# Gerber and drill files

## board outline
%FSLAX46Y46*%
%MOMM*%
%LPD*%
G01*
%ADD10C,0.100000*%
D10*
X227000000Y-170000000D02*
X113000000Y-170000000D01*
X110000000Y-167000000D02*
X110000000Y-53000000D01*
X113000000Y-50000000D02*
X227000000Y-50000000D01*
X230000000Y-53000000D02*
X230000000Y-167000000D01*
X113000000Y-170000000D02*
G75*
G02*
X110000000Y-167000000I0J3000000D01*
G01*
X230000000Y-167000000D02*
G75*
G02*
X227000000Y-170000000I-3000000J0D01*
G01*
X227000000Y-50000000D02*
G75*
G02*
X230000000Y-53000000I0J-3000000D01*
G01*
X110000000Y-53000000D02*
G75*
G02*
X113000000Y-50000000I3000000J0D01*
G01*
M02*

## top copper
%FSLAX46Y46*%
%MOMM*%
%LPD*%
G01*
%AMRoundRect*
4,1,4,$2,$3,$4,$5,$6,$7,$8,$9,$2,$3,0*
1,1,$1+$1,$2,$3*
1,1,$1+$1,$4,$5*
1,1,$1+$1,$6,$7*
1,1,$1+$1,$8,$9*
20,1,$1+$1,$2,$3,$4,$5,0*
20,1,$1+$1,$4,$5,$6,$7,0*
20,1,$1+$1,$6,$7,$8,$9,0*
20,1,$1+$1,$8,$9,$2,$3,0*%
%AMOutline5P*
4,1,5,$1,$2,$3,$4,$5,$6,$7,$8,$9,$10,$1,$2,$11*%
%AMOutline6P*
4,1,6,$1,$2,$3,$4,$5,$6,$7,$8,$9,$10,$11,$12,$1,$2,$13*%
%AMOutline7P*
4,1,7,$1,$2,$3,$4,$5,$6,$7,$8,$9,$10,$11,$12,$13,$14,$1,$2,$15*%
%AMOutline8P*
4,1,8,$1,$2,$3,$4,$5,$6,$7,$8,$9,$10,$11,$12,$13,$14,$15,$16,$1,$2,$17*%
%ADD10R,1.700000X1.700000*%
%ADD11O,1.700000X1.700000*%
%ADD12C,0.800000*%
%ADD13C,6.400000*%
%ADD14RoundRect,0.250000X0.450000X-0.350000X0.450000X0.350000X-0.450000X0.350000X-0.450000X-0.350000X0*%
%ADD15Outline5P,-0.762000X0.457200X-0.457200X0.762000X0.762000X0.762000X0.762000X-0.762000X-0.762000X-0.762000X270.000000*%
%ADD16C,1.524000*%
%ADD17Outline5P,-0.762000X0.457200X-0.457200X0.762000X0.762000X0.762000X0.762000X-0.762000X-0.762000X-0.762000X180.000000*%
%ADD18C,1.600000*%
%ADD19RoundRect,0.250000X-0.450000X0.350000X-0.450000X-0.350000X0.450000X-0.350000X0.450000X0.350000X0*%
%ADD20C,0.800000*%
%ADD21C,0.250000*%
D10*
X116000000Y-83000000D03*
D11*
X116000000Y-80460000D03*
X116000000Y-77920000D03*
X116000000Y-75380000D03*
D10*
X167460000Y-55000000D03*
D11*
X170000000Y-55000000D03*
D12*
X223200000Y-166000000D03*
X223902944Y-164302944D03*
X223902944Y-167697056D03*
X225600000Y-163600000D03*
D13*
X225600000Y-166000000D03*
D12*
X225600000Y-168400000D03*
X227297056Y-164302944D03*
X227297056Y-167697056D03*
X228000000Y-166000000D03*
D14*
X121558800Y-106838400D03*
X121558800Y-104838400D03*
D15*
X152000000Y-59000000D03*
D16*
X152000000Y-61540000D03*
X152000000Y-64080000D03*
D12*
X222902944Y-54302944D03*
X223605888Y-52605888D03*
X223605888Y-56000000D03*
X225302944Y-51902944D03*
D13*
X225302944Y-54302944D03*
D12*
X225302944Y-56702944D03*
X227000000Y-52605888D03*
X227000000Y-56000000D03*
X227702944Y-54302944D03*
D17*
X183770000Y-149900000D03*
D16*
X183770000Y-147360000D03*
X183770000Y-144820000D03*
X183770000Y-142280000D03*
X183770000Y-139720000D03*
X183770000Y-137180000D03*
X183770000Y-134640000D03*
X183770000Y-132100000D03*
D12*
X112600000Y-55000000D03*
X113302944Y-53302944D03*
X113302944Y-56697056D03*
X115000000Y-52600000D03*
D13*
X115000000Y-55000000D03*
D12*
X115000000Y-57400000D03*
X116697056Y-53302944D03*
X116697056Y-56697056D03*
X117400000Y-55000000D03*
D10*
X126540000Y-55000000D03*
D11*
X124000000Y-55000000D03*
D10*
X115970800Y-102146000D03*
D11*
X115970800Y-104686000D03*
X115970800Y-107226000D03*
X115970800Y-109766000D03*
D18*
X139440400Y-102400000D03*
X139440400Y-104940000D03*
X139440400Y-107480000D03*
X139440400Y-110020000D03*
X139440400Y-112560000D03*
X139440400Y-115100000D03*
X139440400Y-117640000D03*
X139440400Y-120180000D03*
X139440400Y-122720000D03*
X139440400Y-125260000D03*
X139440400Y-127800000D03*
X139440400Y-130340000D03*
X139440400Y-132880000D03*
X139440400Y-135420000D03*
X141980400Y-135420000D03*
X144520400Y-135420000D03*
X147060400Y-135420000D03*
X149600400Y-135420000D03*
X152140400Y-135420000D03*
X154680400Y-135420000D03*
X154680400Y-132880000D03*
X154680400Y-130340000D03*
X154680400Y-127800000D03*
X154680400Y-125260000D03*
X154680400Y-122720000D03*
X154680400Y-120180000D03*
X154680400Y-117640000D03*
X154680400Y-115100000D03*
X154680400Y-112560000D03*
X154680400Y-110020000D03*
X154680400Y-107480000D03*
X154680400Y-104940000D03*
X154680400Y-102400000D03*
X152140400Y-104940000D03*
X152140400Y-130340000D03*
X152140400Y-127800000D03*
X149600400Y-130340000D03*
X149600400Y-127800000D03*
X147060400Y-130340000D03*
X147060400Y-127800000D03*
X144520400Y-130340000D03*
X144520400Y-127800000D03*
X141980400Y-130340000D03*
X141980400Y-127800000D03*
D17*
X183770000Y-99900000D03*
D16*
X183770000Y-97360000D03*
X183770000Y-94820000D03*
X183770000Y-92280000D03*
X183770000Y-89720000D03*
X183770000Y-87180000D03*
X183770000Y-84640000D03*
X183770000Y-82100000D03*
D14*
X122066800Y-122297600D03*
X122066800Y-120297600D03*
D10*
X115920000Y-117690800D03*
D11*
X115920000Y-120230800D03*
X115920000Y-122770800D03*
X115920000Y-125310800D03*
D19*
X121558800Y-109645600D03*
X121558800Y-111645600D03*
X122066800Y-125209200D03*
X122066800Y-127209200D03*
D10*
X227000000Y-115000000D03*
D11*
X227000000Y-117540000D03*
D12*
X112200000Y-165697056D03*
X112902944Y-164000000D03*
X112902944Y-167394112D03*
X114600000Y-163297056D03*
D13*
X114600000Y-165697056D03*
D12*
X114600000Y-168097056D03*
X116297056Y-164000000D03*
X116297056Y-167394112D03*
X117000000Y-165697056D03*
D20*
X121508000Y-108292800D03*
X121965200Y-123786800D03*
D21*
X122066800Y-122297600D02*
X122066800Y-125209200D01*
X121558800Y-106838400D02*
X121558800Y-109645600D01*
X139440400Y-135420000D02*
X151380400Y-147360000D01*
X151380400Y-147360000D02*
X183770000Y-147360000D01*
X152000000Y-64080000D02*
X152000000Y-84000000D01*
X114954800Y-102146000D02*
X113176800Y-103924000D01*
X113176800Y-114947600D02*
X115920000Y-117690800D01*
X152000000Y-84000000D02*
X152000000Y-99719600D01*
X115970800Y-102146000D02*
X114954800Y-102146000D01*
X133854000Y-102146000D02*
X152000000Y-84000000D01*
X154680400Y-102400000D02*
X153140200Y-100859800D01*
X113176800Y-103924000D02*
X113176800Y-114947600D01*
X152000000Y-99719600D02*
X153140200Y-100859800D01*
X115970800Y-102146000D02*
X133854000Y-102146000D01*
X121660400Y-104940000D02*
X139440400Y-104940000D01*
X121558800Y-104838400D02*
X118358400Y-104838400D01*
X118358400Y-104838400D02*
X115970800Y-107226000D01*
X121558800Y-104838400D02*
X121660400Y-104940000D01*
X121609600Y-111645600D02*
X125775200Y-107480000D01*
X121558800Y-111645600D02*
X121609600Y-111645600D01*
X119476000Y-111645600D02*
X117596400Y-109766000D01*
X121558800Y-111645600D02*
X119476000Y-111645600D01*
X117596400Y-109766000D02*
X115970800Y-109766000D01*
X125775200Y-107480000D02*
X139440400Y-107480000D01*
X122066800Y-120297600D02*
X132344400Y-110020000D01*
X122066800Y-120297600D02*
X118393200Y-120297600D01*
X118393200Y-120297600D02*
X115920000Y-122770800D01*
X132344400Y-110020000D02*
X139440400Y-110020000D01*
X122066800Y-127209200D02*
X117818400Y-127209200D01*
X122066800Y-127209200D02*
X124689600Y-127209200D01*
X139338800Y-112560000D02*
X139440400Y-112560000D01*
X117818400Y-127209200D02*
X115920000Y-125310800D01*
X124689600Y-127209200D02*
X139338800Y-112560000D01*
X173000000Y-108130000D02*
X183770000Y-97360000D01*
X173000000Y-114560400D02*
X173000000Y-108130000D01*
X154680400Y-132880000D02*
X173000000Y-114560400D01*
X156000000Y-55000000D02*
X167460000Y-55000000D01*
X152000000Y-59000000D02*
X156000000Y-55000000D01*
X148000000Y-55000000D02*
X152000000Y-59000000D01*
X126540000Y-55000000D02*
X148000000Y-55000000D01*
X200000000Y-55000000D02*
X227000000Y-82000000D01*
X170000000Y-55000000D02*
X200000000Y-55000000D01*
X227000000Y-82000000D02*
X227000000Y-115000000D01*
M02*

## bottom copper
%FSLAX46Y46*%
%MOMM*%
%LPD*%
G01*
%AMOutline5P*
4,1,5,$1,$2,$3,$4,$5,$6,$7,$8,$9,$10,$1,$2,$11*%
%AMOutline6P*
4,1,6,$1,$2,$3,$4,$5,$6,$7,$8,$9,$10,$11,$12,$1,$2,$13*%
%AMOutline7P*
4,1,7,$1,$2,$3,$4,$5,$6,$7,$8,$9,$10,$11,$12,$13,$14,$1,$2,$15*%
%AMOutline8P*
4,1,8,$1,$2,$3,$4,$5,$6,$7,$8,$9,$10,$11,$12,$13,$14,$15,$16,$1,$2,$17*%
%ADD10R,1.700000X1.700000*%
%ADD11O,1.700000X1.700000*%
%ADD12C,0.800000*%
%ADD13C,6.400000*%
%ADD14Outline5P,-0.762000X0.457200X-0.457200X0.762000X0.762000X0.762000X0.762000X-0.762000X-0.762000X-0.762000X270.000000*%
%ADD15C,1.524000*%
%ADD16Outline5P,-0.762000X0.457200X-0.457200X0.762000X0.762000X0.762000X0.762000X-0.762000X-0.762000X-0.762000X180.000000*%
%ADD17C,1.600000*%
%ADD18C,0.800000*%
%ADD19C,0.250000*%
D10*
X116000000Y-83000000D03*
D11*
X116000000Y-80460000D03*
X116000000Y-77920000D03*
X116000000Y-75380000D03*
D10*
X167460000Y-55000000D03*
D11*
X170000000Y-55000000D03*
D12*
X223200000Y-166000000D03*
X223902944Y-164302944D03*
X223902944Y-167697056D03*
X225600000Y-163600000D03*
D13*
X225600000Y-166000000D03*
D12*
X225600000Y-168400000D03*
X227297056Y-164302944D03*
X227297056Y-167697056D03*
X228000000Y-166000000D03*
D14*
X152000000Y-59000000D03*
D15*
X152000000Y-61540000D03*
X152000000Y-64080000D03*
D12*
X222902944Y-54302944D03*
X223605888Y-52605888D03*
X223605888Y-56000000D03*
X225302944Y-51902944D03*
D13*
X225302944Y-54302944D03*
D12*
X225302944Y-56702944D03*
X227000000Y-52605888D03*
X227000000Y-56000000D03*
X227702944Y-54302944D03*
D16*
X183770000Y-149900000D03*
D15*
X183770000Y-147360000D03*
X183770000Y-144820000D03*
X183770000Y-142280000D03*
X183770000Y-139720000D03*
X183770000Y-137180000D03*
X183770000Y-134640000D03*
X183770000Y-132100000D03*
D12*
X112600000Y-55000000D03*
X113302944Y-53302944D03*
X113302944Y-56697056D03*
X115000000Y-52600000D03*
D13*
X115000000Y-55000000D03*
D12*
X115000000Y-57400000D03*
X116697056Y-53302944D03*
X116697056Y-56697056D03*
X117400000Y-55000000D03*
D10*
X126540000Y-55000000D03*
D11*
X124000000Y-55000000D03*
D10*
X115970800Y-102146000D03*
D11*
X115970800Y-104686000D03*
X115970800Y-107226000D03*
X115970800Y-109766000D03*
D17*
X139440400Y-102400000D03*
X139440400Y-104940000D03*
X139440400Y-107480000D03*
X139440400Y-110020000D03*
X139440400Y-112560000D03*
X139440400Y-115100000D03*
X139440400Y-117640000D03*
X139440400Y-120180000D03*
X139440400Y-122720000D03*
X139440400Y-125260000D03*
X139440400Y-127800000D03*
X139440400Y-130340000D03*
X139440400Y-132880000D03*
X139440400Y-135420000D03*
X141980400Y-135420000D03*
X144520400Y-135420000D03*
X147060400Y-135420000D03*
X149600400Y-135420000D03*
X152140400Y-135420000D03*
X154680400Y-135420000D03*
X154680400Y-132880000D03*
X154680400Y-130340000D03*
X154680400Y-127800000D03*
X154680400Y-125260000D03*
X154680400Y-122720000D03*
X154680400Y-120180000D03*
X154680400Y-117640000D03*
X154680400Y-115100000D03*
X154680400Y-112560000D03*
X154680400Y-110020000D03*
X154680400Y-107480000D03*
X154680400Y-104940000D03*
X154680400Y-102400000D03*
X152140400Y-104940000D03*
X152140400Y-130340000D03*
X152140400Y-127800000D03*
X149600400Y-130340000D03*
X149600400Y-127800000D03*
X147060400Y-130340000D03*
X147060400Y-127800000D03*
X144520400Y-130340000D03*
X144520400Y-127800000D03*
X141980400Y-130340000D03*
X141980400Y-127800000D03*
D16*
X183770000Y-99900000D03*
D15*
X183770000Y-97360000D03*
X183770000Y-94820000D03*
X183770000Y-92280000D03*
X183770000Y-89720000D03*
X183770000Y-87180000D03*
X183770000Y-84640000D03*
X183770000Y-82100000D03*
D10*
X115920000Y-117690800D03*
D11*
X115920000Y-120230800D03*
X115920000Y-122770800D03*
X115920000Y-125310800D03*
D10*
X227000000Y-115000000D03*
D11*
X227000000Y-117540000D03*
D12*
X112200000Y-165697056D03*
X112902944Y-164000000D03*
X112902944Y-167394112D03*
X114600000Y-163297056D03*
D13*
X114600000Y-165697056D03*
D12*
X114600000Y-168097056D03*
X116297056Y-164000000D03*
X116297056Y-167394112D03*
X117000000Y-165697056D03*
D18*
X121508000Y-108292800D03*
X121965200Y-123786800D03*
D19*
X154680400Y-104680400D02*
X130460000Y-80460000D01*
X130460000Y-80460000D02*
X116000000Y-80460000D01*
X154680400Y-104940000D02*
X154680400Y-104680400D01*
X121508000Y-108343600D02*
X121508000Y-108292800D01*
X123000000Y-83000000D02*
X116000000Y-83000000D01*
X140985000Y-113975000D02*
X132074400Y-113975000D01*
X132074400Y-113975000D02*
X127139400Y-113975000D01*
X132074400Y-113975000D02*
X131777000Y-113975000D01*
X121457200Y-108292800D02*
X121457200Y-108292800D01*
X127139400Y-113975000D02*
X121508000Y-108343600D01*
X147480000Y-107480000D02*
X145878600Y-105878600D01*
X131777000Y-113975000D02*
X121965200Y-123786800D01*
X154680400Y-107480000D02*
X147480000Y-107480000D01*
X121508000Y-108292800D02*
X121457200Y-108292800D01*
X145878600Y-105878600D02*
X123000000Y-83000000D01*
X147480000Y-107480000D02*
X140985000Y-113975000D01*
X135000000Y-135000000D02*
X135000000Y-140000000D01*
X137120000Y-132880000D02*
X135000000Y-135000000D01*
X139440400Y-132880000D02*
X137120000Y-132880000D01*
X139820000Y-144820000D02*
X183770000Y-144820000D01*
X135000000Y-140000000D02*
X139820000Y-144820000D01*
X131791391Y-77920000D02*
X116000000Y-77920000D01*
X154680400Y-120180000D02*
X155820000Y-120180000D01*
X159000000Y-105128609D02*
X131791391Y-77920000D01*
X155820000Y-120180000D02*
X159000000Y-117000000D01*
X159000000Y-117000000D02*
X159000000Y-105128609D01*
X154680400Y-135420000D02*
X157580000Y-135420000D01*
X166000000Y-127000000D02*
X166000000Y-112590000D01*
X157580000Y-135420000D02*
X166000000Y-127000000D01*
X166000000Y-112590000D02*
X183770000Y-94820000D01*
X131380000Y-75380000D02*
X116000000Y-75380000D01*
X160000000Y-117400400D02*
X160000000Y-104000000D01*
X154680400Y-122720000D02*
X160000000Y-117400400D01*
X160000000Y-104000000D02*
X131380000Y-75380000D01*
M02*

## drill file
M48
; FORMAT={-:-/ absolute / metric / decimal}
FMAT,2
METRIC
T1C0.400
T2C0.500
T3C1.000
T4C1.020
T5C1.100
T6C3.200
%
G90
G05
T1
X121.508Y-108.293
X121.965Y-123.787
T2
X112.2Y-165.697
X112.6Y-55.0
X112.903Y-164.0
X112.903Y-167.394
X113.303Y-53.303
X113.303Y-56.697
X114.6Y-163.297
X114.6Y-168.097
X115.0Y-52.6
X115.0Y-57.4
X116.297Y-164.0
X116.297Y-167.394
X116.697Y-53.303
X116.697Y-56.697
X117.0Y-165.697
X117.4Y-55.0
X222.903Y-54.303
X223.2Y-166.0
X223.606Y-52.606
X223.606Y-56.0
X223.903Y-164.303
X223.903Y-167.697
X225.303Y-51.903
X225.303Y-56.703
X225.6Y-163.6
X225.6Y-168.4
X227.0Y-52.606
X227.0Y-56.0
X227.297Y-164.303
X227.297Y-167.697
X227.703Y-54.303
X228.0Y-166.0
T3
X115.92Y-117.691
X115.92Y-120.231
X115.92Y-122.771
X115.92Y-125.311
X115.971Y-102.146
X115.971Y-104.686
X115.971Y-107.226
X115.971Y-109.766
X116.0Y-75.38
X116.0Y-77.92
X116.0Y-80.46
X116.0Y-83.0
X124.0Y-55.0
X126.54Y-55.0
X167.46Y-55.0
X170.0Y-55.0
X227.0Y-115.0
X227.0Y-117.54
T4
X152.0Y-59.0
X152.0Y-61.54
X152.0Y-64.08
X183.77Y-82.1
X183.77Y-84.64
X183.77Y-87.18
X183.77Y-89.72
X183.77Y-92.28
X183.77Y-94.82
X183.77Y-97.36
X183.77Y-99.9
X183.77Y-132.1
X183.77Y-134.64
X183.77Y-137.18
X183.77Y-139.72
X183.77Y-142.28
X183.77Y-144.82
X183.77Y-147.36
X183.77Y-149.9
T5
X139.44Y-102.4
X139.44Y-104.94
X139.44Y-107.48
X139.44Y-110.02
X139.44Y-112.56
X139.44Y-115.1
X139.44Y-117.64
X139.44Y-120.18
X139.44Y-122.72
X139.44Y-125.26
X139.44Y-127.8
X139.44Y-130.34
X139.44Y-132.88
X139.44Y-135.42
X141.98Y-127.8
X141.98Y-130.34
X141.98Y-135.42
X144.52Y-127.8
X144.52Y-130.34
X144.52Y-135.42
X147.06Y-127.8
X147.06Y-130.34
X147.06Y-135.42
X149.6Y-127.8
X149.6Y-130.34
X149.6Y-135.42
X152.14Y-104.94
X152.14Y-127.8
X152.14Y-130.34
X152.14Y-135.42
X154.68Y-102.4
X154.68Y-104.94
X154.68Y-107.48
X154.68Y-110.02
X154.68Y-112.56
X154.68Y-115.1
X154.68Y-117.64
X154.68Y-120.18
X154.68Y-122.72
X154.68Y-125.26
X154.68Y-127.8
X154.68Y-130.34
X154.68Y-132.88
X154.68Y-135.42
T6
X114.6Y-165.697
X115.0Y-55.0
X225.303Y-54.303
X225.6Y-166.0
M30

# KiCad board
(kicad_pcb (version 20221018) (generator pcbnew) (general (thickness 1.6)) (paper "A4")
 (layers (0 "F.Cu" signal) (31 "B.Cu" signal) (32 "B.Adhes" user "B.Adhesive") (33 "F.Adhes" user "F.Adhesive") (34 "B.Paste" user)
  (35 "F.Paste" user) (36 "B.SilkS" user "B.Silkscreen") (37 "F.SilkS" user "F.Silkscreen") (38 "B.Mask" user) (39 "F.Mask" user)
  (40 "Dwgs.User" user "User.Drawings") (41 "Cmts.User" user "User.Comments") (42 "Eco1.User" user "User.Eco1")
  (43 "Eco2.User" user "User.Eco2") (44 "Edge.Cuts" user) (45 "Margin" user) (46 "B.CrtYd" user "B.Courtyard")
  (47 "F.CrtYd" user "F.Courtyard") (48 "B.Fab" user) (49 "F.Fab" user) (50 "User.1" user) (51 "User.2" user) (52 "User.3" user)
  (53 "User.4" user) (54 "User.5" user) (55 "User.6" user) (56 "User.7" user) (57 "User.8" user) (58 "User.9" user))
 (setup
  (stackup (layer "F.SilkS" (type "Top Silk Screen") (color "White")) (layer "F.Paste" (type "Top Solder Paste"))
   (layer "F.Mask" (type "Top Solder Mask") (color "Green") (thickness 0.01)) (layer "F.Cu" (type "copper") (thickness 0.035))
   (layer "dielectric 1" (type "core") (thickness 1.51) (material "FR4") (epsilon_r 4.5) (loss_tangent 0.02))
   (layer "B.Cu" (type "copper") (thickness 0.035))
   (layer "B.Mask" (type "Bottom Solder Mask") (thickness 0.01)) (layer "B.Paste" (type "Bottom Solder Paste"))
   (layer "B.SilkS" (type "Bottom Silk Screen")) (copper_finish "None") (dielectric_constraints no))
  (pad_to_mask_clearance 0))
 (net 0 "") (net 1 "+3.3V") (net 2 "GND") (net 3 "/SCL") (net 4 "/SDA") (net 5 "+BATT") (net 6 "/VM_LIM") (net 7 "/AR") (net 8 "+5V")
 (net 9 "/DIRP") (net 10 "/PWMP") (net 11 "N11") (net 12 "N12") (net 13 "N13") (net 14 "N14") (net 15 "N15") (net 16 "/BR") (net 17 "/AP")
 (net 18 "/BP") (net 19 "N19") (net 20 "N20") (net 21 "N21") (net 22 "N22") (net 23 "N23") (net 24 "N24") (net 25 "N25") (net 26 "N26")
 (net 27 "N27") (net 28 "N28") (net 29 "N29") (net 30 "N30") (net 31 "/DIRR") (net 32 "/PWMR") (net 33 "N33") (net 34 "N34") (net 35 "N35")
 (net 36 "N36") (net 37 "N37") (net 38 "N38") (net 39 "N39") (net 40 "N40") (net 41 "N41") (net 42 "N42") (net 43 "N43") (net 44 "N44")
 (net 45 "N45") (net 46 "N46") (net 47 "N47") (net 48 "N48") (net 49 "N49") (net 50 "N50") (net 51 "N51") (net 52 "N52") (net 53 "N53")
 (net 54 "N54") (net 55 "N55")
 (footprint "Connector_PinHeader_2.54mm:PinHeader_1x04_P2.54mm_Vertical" (layer "F.Cu") (at 116 83 180)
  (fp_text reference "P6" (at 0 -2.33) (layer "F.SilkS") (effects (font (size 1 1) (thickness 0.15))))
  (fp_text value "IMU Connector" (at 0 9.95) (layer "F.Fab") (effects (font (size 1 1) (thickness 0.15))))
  (pad "1" thru_hole rect (at 0 0 180) (size 1.7 1.7) (drill 1) (layers "*.Cu" "*.Mask") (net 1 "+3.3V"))
  (pad "2" thru_hole oval (at 0 2.54 180) (size 1.7 1.7) (drill 1) (layers "*.Cu" "*.Mask") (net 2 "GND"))
  (pad "3" thru_hole oval (at 0 5.08 180) (size 1.7 1.7) (drill 1) (layers "*.Cu" "*.Mask") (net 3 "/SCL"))
  (pad "4" thru_hole oval (at 0 7.62 180) (size 1.7 1.7) (drill 1) (layers "*.Cu" "*.Mask") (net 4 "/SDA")))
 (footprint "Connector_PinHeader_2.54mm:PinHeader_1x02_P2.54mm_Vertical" (layer "F.Cu") (at 167.46 55 90)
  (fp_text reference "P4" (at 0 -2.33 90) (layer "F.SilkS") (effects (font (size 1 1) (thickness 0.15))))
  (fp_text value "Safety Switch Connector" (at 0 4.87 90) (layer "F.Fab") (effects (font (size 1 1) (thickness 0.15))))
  (pad "1" thru_hole rect (at 0 0 90) (size 1.7 1.7) (drill 1) (layers "*.Cu" "*.Mask") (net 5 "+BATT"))
  (pad "2" thru_hole oval (at 0 2.54 90) (size 1.7 1.7) (drill 1) (layers "*.Cu" "*.Mask") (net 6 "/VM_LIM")))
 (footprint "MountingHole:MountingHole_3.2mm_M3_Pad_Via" (layer "F.Cu") (at 225.6 166)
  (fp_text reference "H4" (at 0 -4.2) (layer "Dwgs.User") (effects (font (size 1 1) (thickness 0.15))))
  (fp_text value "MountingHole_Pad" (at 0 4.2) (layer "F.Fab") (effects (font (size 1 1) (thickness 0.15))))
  (pad "1" thru_hole circle (at -2.4 0) (size 0.8 0.8) (drill 0.5) (layers "*.Cu" "*.Mask") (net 2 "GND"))
  (pad "1" thru_hole circle (at -1.697056 -1.697056) (size 0.8 0.8) (drill 0.5) (layers "*.Cu" "*.Mask") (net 2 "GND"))
  (pad "1" thru_hole circle (at -1.697056 1.697056) (size 0.8 0.8) (drill 0.5) (layers "*.Cu" "*.Mask") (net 2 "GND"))
  (pad "1" thru_hole circle (at 0 -2.4) (size 0.8 0.8) (drill 0.5) (layers "*.Cu" "*.Mask") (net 2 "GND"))
  (pad "1" thru_hole circle (at 0 0) (size 6.4 6.4) (drill 3.2) (layers "*.Cu" "*.Mask") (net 2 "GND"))
  (pad "1" thru_hole circle (at 0 2.4) (size 0.8 0.8) (drill 0.5) (layers "*.Cu" "*.Mask") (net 2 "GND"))
  (pad "1" thru_hole circle (at 1.697056 -1.697056) (size 0.8 0.8) (drill 0.5) (layers "*.Cu" "*.Mask") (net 2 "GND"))
  (pad "1" thru_hole circle (at 1.697056 1.697056) (size 0.8 0.8) (drill 0.5) (layers "*.Cu" "*.Mask") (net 2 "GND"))
  (pad "1" thru_hole circle (at 2.4 0) (size 0.8 0.8) (drill 0.5) (layers "*.Cu" "*.Mask") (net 2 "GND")))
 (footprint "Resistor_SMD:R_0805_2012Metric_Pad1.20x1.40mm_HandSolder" (layer "F.Cu") (at 121.5588 105.8384 90)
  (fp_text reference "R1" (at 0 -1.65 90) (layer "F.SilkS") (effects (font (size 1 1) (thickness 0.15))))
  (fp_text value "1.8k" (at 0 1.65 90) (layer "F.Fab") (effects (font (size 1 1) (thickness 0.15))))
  (pad "1" smd roundrect (at -1 0 90) (size 1.2 1.4) (layers "F.Cu" "F.Paste" "F.Mask") (roundrect_rratio 0.208333) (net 1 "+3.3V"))
  (pad "2" smd roundrect (at 1 0 90) (size 1.2 1.4) (layers "F.Cu" "F.Paste" "F.Mask") (roundrect_rratio 0.208333) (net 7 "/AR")))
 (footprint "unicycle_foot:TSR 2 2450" (layer "F.Cu") (at 151.86 61.58 -90)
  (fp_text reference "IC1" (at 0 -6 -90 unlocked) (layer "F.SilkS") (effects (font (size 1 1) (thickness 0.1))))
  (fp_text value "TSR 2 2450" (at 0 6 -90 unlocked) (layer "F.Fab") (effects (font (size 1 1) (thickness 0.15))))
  (pad "1" thru_hole roundrect (at -2.58 -0.14 270) (size 1.524 1.524) (drill 1.02) (layers "*.Cu" "*.Mask") (roundrect_rratio 0)
   (chamfer_ratio 0.2) (chamfer top_left) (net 5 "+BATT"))
  (pad "2" thru_hole circle (at -0.04 -0.14 270) (size 1.524 1.524) (drill 1.02) (layers "*.Cu" "*.Mask") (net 2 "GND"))
  (pad "3" thru_hole circle (at 2.5 -0.14 270) (size 1.524 1.524) (drill 1.02) (layers "*.Cu" "*.Mask") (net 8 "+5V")))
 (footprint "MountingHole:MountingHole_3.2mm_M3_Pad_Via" (layer "F.Cu") (at 225.302944 54.302944)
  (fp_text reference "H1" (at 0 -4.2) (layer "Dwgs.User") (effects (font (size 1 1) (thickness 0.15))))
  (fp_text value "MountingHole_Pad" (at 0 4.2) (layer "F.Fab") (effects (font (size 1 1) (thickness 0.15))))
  (pad "1" thru_hole circle (at -2.4 0) (size 0.8 0.8) (drill 0.5) (layers "*.Cu" "*.Mask") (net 2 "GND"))
  (pad "1" thru_hole circle (at -1.697056 -1.697056) (size 0.8 0.8) (drill 0.5) (layers "*.Cu" "*.Mask") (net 2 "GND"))
  (pad "1" thru_hole circle (at -1.697056 1.697056) (size 0.8 0.8) (drill 0.5) (layers "*.Cu" "*.Mask") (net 2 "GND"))
  (pad "1" thru_hole circle (at 0 -2.4) (size 0.8 0.8) (drill 0.5) (layers "*.Cu" "*.Mask") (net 2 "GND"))
  (pad "1" thru_hole circle (at 0 0) (size 6.4 6.4) (drill 3.2) (layers "*.Cu" "*.Mask") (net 2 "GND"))
  (pad "1" thru_hole circle (at 0 2.4) (size 0.8 0.8) (drill 0.5) (layers "*.Cu" "*.Mask") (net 2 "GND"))
  (pad "1" thru_hole circle (at 1.697056 -1.697056) (size 0.8 0.8) (drill 0.5) (layers "*.Cu" "*.Mask") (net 2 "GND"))
  (pad "1" thru_hole circle (at 1.697056 1.697056) (size 0.8 0.8) (drill 0.5) (layers "*.Cu" "*.Mask") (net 2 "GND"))
  (pad "1" thru_hole circle (at 2.4 0) (size 0.8 0.8) (drill 0.5) (layers "*.Cu" "*.Mask") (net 2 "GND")))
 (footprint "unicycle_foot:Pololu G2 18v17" (layer "F.Cu") (at 199 141 180)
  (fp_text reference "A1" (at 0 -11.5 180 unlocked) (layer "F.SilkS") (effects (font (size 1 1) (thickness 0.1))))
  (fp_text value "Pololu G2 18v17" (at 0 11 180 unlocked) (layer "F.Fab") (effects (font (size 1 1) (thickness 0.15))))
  (pad "1" thru_hole roundrect (at 15.23 -8.9 180) (size 1.524 1.524) (drill 1.02) (layers "*.Cu" "*.Mask") (roundrect_rratio 0)
   (chamfer_ratio 0.2) (chamfer top_left) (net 2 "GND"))
  (pad "2" thru_hole circle (at 15.23 -6.36 180) (size 1.524 1.524) (drill 1.02) (layers "*.Cu" "*.Mask") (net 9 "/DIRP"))
  (pad "3" thru_hole circle (at 15.23 -3.82 180) (size 1.524 1.524) (drill 1.02) (layers "*.Cu" "*.Mask") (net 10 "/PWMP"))
  (pad "4" thru_hole circle (at 15.23 -1.28 180) (size 1.524 1.524) (drill 1.02) (layers "*.Cu" "*.Mask") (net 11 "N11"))
  (pad "5" thru_hole circle (at 15.23 1.28 180) (size 1.524 1.524) (drill 1.02) (layers "*.Cu" "*.Mask") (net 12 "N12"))
  (pad "6" thru_hole circle (at 15.23 3.82 180) (size 1.524 1.524) (drill 1.02) (layers "*.Cu" "*.Mask") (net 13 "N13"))
  (pad "7" thru_hole circle (at 15.23 6.36 180) (size 1.524 1.524) (drill 1.02) (layers "*.Cu" "*.Mask") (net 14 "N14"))
  (pad "8" thru_hole circle (at 15.23 8.9 180) (size 1.524 1.524) (drill 1.02) (layers "*.Cu" "*.Mask") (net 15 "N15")))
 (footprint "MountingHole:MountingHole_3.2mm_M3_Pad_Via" (layer "F.Cu") (at 115 55)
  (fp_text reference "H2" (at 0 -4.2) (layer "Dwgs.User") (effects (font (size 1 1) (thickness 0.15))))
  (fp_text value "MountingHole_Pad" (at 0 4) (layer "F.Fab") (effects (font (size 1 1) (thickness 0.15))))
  (pad "1" thru_hole circle (at -2.4 0) (size 0.8 0.8) (drill 0.5) (layers "*.Cu" "*.Mask") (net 2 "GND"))
  (pad "1" thru_hole circle (at -1.697056 -1.697056) (size 0.8 0.8) (drill 0.5) (layers "*.Cu" "*.Mask") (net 2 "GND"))
  (pad "1" thru_hole circle (at -1.697056 1.697056) (size 0.8 0.8) (drill 0.5) (layers "*.Cu" "*.Mask") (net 2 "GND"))
  (pad "1" thru_hole circle (at 0 -2.4) (size 0.8 0.8) (drill 0.5) (layers "*.Cu" "*.Mask") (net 2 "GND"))
  (pad "1" thru_hole circle (at 0 0) (size 6.4 6.4) (drill 3.2) (layers "*.Cu" "*.Mask") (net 2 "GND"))
  (pad "1" thru_hole circle (at 0 2.4) (size 0.8 0.8) (drill 0.5) (layers "*.Cu" "*.Mask") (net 2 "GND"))
  (pad "1" thru_hole circle (at 1.697056 -1.697056) (size 0.8 0.8) (drill 0.5) (layers "*.Cu" "*.Mask") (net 2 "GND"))
  (pad "1" thru_hole circle (at 1.697056 1.697056) (size 0.8 0.8) (drill 0.5) (layers "*.Cu" "*.Mask") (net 2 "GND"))
  (pad "1" thru_hole circle (at 2.4 0) (size 0.8 0.8) (drill 0.5) (layers "*.Cu" "*.Mask") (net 2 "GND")))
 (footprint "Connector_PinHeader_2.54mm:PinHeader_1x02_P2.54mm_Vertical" (layer "F.Cu") (at 126.54 55 -90)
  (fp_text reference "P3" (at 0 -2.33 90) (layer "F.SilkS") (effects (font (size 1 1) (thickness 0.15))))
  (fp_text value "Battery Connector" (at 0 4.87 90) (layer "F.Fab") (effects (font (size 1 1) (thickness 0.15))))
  (pad "1" thru_hole rect (at 0 0 270) (size 1.7 1.7) (drill 1) (layers "*.Cu" "*.Mask") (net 5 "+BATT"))
  (pad "2" thru_hole oval (at 0 2.54 270) (size 1.7 1.7) (drill 1) (layers "*.Cu" "*.Mask") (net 2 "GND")))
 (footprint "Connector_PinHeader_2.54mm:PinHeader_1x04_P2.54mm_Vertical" (layer "F.Cu") (at 115.9708 102.146)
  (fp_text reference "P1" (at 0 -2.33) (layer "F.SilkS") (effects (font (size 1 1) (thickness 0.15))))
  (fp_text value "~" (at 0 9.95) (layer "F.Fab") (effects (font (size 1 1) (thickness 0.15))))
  (pad "1" thru_hole rect (at 0 0) (size 1.7 1.7) (drill 1) (layers "*.Cu" "*.Mask") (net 8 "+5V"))
  (pad "2" thru_hole oval (at 0 2.54) (size 1.7 1.7) (drill 1) (layers "*.Cu" "*.Mask") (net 2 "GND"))
  (pad "3" thru_hole oval (at 0 5.08) (size 1.7 1.7) (drill 1) (layers "*.Cu" "*.Mask") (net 7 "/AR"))
  (pad "4" thru_hole oval (at 0 7.62) (size 1.7 1.7) (drill 1) (layers "*.Cu" "*.Mask") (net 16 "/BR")))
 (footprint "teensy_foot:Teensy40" (layer "F.Cu") (at 147.0604 118.91 -90)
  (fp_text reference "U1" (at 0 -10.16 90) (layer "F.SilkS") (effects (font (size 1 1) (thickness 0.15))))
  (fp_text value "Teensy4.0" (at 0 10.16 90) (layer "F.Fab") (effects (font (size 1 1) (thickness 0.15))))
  (pad "1" thru_hole circle (at -16.51 7.62 270) (size 1.6 1.6) (drill 1.1) (layers "*.Cu" "*.Mask") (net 2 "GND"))
  (pad "2" thru_hole circle (at -13.97 7.62 270) (size 1.6 1.6) (drill 1.1) (layers "*.Cu" "*.Mask") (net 7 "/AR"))
  (pad "3" thru_hole circle (at -11.43 7.62 270) (size 1.6 1.6) (drill 1.1) (layers "*.Cu" "*.Mask") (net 16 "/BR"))
  (pad "4" thru_hole circle (at -8.89 7.62 270) (size 1.6 1.6) (drill 1.1) (layers "*.Cu" "*.Mask") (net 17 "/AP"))
  (pad "5" thru_hole circle (at -6.35 7.62 270) (size 1.6 1.6) (drill 1.1) (layers "*.Cu" "*.Mask") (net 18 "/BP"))
  (pad "6" thru_hole circle (at -3.81 7.62 270) (size 1.6 1.6) (drill 1.1) (layers "*.Cu" "*.Mask") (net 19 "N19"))
  (pad "7" thru_hole circle (at -1.27 7.62 270) (size 1.6 1.6) (drill 1.1) (layers "*.Cu" "*.Mask") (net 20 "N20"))
  (pad "8" thru_hole circle (at 1.27 7.62 270) (size 1.6 1.6) (drill 1.1) (layers "*.Cu" "*.Mask") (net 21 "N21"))
  (pad "9" thru_hole circle (at 3.81 7.62 270) (size 1.6 1.6) (drill 1.1) (layers "*.Cu" "*.Mask") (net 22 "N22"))
  (pad "10" thru_hole circle (at 6.35 7.62 270) (size 1.6 1.6) (drill 1.1) (layers "*.Cu" "*.Mask") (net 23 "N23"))
  (pad "11" thru_hole circle (at 8.89 7.62 270) (size 1.6 1.6) (drill 1.1) (layers "*.Cu" "*.Mask") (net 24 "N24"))
  (pad "12" thru_hole circle (at 11.43 7.62 270) (size 1.6 1.6) (drill 1.1) (layers "*.Cu" "*.Mask") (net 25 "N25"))
  (pad "13" thru_hole circle (at 13.97 7.62 270) (size 1.6 1.6) (drill 1.1) (layers "*.Cu" "*.Mask") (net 10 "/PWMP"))
  (pad "14" thru_hole circle (at 16.51 7.62 270) (size 1.6 1.6) (drill 1.1) (layers "*.Cu" "*.Mask") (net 9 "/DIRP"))
  (pad "15" thru_hole circle (at 16.51 5.08 270) (size 1.6 1.6) (drill 1.1) (layers "*.Cu" "*.Mask") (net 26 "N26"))
  (pad "16" thru_hole circle (at 16.51 2.54 270) (size 1.6 1.6) (drill 1.1) (layers "*.Cu" "*.Mask") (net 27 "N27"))
  (pad "17" thru_hole circle (at 16.51 0 270) (size 1.6 1.6) (drill 1.1) (layers "*.Cu" "*.Mask") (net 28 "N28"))
  (pad "18" thru_hole circle (at 16.51 -2.54 270) (size 1.6 1.6) (drill 1.1) (layers "*.Cu" "*.Mask") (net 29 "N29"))
  (pad "19" thru_hole circle (at 16.51 -5.08 270) (size 1.6 1.6) (drill 1.1) (layers "*.Cu" "*.Mask") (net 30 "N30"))
  (pad "20" thru_hole circle (at 16.51 -7.62 270) (size 1.6 1.6) (drill 1.1) (layers "*.Cu" "*.Mask") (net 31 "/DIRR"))
  (pad "21" thru_hole circle (at 13.97 -7.62 270) (size 1.6 1.6) (drill 1.1) (layers "*.Cu" "*.Mask") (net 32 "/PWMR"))
  (pad "22" thru_hole circle (at 11.43 -7.62 270) (size 1.6 1.6) (drill 1.1) (layers "*.Cu" "*.Mask") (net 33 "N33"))
  (pad "23" thru_hole circle (at 8.89 -7.62 270) (size 1.6 1.6) (drill 1.1) (layers "*.Cu" "*.Mask") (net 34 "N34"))
  (pad "24" thru_hole circle (at 6.35 -7.62 270) (size 1.6 1.6) (drill 1.1) (layers "*.Cu" "*.Mask") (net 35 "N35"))
  (pad "25" thru_hole circle (at 3.81 -7.62 270) (size 1.6 1.6) (drill 1.1) (layers "*.Cu" "*.Mask") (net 4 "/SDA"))
  (pad "26" thru_hole circle (at 1.27 -7.62 270) (size 1.6 1.6) (drill 1.1) (layers "*.Cu" "*.Mask") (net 3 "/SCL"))
  (pad "27" thru_hole circle (at -1.27 -7.62 270) (size 1.6 1.6) (drill 1.1) (layers "*.Cu" "*.Mask") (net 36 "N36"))
  (pad "28" thru_hole circle (at -3.81 -7.62 270) (size 1.6 1.6) (drill 1.1) (layers "*.Cu" "*.Mask") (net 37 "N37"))
  (pad "29" thru_hole circle (at -6.35 -7.62 270) (size 1.6 1.6) (drill 1.1) (layers "*.Cu" "*.Mask") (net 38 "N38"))
  (pad "30" thru_hole circle (at -8.89 -7.62 270) (size 1.6 1.6) (drill 1.1) (layers "*.Cu" "*.Mask") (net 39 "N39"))
  (pad "31" thru_hole circle (at -11.43 -7.62 270) (size 1.6 1.6) (drill 1.1) (layers "*.Cu" "*.Mask") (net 1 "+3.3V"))
  (pad "32" thru_hole circle (at -13.97 -7.62 270) (size 1.6 1.6) (drill 1.1) (layers "*.Cu" "*.Mask") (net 2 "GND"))
  (pad "33" thru_hole circle (at -16.51 -7.62 270) (size 1.6 1.6) (drill 1.1) (layers "*.Cu" "*.Mask") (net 8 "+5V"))
  (pad "34" thru_hole circle (at -13.97 -5.08 270) (size 1.6 1.6) (drill 1.1) (layers "*.Cu" "*.Mask") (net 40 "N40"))
  (pad "35" thru_hole circle (at 11.43 -5.08 270) (size 1.6 1.6) (drill 1.1) (layers "*.Cu" "*.Mask") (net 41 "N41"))
  (pad "36" thru_hole circle (at 8.89 -5.08 270) (size 1.6 1.6) (drill 1.1) (layers "*.Cu" "*.Mask") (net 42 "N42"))
  (pad "37" thru_hole circle (at 11.43 -2.54 270) (size 1.6 1.6) (drill 1.1) (layers "*.Cu" "*.Mask") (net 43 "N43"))
  (pad "38" thru_hole circle (at 8.89 -2.54 270) (size 1.6 1.6) (drill 1.1) (layers "*.Cu" "*.Mask") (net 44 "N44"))
  (pad "39" thru_hole circle (at 11.43 0 270) (size 1.6 1.6) (drill 1.1) (layers "*.Cu" "*.Mask") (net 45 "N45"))
  (pad "40" thru_hole circle (at 8.89 0 270) (size 1.6 1.6) (drill 1.1) (layers "*.Cu" "*.Mask") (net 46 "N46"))
  (pad "41" thru_hole circle (at 11.43 2.54 270) (size 1.6 1.6) (drill 1.1) (layers "*.Cu" "*.Mask") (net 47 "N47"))
  (pad "42" thru_hole circle (at 8.89 2.54 270) (size 1.6 1.6) (drill 1.1) (layers "*.Cu" "*.Mask") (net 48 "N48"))
  (pad "43" thru_hole circle (at 11.43 5.08 270) (size 1.6 1.6) (drill 1.1) (layers "*.Cu" "*.Mask") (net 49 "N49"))
  (pad "44" thru_hole circle (at 8.89 5.08 270) (size 1.6 1.6) (drill 1.1) (layers "*.Cu" "*.Mask") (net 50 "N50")))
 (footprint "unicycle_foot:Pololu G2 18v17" (layer "F.Cu") (at 199 91 180)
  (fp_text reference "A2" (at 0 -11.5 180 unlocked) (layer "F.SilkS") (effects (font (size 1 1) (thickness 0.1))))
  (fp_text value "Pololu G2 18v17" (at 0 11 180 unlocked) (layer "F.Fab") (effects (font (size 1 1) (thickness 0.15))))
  (pad "1" thru_hole roundrect (at 15.23 -8.9 180) (size 1.524 1.524) (drill 1.02) (layers "*.Cu" "*.Mask") (roundrect_rratio 0)
   (chamfer_ratio 0.2) (chamfer top_left) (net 2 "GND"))
  (pad "2" thru_hole circle (at 15.23 -6.36 180) (size 1.524 1.524) (drill 1.02) (layers "*.Cu" "*.Mask") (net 32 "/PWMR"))
  (pad "3" thru_hole circle (at 15.23 -3.82 180) (size 1.524 1.524) (drill 1.02) (layers "*.Cu" "*.Mask") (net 31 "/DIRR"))
  (pad "4" thru_hole circle (at 15.23 -1.28 180) (size 1.524 1.524) (drill 1.02) (layers "*.Cu" "*.Mask") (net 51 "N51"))
  (pad "5" thru_hole circle (at 15.23 1.28 180) (size 1.524 1.524) (drill 1.02) (layers "*.Cu" "*.Mask") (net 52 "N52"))
  (pad "6" thru_hole circle (at 15.23 3.82 180) (size 1.524 1.524) (drill 1.02) (layers "*.Cu" "*.Mask") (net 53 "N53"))
  (pad "7" thru_hole circle (at 15.23 6.36 180) (size 1.524 1.524) (drill 1.02) (layers "*.Cu" "*.Mask") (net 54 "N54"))
  (pad "8" thru_hole circle (at 15.23 8.9 180) (size 1.524 1.524) (drill 1.02) (layers "*.Cu" "*.Mask") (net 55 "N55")))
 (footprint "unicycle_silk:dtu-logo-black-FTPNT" (layer "F.Cu") (at 214 160)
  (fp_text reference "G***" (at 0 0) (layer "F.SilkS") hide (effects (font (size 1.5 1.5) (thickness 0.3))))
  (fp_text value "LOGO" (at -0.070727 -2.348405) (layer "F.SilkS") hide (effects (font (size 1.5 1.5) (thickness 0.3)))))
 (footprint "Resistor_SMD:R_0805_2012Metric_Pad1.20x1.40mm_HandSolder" (layer "F.Cu") (at 122.0668 121.2976 90)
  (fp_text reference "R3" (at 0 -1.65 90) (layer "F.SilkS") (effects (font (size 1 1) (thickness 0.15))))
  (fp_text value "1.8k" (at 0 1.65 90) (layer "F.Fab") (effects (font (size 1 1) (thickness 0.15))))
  (pad "1" smd roundrect (at -1 0 90) (size 1.2 1.4) (layers "F.Cu" "F.Paste" "F.Mask") (roundrect_rratio 0.208333) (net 1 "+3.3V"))
  (pad "2" smd roundrect (at 1 0 90) (size 1.2 1.4) (layers "F.Cu" "F.Paste" "F.Mask") (roundrect_rratio 0.208333) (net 17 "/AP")))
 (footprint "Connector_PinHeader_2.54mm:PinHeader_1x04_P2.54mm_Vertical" (layer "F.Cu") (at 115.92 117.6908)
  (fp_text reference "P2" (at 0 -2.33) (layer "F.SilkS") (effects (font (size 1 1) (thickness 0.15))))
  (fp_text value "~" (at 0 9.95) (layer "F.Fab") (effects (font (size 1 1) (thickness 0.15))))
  (pad "1" thru_hole rect (at 0 0) (size 1.7 1.7) (drill 1) (layers "*.Cu" "*.Mask") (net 8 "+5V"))
  (pad "2" thru_hole oval (at 0 2.54) (size 1.7 1.7) (drill 1) (layers "*.Cu" "*.Mask") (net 2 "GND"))
  (pad "3" thru_hole oval (at 0 5.08) (size 1.7 1.7) (drill 1) (layers "*.Cu" "*.Mask") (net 17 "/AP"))
  (pad "4" thru_hole oval (at 0 7.62) (size 1.7 1.7) (drill 1) (layers "*.Cu" "*.Mask") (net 18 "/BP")))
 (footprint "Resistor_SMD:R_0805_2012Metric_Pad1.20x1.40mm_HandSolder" (layer "F.Cu") (at 121.5588 110.6456 -90)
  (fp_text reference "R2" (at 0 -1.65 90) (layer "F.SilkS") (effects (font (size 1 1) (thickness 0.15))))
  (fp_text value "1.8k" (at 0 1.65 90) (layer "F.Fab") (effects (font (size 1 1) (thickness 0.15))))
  (pad "1" smd roundrect (at -1 0 270) (size 1.2 1.4) (layers "F.Cu" "F.Paste" "F.Mask") (roundrect_rratio 0.208333) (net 1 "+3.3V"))
  (pad "2" smd roundrect (at 1 0 270) (size 1.2 1.4) (layers "F.Cu" "F.Paste" "F.Mask") (roundrect_rratio 0.208333) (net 16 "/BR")))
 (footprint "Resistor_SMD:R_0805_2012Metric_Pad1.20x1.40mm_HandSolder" (layer "F.Cu") (at 122.0668 126.2092 -90)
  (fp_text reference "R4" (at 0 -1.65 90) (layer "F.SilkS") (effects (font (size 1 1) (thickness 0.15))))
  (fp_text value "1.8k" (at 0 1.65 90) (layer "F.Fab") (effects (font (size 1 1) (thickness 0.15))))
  (pad "1" smd roundrect (at -1 0 270) (size 1.2 1.4) (layers "F.Cu" "F.Paste" "F.Mask") (roundrect_rratio 0.208333) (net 1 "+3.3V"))
  (pad "2" smd roundrect (at 1 0 270) (size 1.2 1.4) (layers "F.Cu" "F.Paste" "F.Mask") (roundrect_rratio 0.208333) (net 18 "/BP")))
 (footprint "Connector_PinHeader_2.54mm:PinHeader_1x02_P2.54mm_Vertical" (layer "F.Cu") (at 227 115)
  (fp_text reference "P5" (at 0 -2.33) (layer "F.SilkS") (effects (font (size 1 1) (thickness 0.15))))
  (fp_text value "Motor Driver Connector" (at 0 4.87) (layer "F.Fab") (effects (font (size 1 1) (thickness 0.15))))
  (pad "1" thru_hole rect (at 0 0) (size 1.7 1.7) (drill 1) (layers "*.Cu" "*.Mask") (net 6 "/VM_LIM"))
  (pad "2" thru_hole oval (at 0 2.54) (size 1.7 1.7) (drill 1) (layers "*.Cu" "*.Mask") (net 2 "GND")))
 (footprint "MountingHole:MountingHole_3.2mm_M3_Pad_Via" (layer "F.Cu") (at 114.6 165.697056)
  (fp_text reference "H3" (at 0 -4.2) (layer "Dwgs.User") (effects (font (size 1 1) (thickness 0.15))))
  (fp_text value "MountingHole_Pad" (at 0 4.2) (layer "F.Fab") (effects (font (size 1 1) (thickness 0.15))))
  (pad "1" thru_hole circle (at -2.4 0) (size 0.8 0.8) (drill 0.5) (layers "*.Cu" "*.Mask") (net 2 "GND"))
  (pad "1" thru_hole circle (at -1.697056 -1.697056) (size 0.8 0.8) (drill 0.5) (layers "*.Cu" "*.Mask") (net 2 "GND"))
  (pad "1" thru_hole circle (at -1.697056 1.697056) (size 0.8 0.8) (drill 0.5) (layers "*.Cu" "*.Mask") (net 2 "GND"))
  (pad "1" thru_hole circle (at 0 -2.4) (size 0.8 0.8) (drill 0.5) (layers "*.Cu" "*.Mask") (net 2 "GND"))
  (pad "1" thru_hole circle (at 0 0) (size 6.4 6.4) (drill 3.2) (layers "*.Cu" "*.Mask") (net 2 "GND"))
  (pad "1" thru_hole circle (at 0 2.4) (size 0.8 0.8) (drill 0.5) (layers "*.Cu" "*.Mask") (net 2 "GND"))
  (pad "1" thru_hole circle (at 1.697056 -1.697056) (size 0.8 0.8) (drill 0.5) (layers "*.Cu" "*.Mask") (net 2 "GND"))
  (pad "1" thru_hole circle (at 1.697056 1.697056) (size 0.8 0.8) (drill 0.5) (layers "*.Cu" "*.Mask") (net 2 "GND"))
  (pad "1" thru_hole circle (at 2.4 0) (size 0.8 0.8) (drill 0.5) (layers "*.Cu" "*.Mask") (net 2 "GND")))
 (gr_line (start 227 170) (end 113 170) (stroke (width 0.1) (type default)) (layer "Edge.Cuts"))
 (gr_line (start 110 167) (end 110 53) (stroke (width 0.1) (type default)) (layer "Edge.Cuts"))
 (gr_line (start 113 50) (end 227 50) (stroke (width 0.1) (type default)) (layer "Edge.Cuts"))
 (gr_line (start 230 53) (end 230 167) (stroke (width 0.1) (type default)) (layer "Edge.Cuts"))
 (gr_arc (start 113 170) (mid 110.87868 169.12132) (end 110 167) (stroke (width 0.1) (type default)) (layer "Edge.Cuts"))
 (gr_arc (start 230 167) (mid 229.12132 169.12132) (end 227 170) (stroke (width 0.1) (type default)) (layer "Edge.Cuts"))
 (gr_arc (start 227 50) (mid 229.12132 50.87868) (end 230 53) (stroke (width 0.1) (type default)) (layer "Edge.Cuts"))
 (gr_arc (start 110 53) (mid 110.87868 50.87868) (end 113 50) (stroke (width 0.1) (type default)) (layer "Edge.Cuts"))
 (segment (start 154.6804 104.6804) (end 130.46 80.46) (width 0.25) (layer "B.Cu") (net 2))
 (segment (start 130.46 80.46) (end 116 80.46) (width 0.25) (layer "B.Cu") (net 2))
 (segment (start 154.6804 104.94) (end 154.6804 104.6804) (width 0.25) (layer "B.Cu") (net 2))
 (segment (start 122.0668 122.2976) (end 122.0668 125.2092) (width 0.25) (layer "F.Cu") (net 1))
 (segment (start 121.5588 106.8384) (end 121.5588 109.6456) (width 0.25) (layer "F.Cu") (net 1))
 (via (at 121.508 108.2928) (size 0.8) (drill 0.4) (layers "F.Cu" "B.Cu") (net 1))
 (via (at 121.9652 123.7868) (size 0.8) (drill 0.4) (layers "F.Cu" "B.Cu") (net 1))
 (segment (start 121.508 108.3436) (end 121.508 108.2928) (width 0.25) (layer "B.Cu") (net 1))
 (segment (start 123 83) (end 116 83) (width 0.25) (layer "B.Cu") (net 1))
 (segment (start 140.985 113.975) (end 132.0744 113.975) (width 0.25) (layer "B.Cu") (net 1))
 (segment (start 132.0744 113.975) (end 127.1394 113.975) (width 0.25) (layer "B.Cu") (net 1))
 (segment (start 132.0744 113.975) (end 131.777 113.975) (width 0.25) (layer "B.Cu") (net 1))
 (segment (start 121.4572 108.2928) (end 121.4572 108.2928) (width 0.25) (layer "B.Cu") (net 1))
 (segment (start 127.1394 113.975) (end 121.508 108.3436) (width 0.25) (layer "B.Cu") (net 1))
 (segment (start 147.48 107.48) (end 145.8786 105.8786) (width 0.25) (layer "B.Cu") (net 1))
 (segment (start 131.777 113.975) (end 121.9652 123.7868) (width 0.25) (layer "B.Cu") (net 1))
 (segment (start 154.6804 107.48) (end 147.48 107.48) (width 0.25) (layer "B.Cu") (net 1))
 (segment (start 121.508 108.2928) (end 121.4572 108.2928) (width 0.25) (layer "B.Cu") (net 1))
 (segment (start 145.8786 105.8786) (end 123 83) (width 0.25) (layer "B.Cu") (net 1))
 (segment (start 147.48 107.48) (end 140.985 113.975) (width 0.25) (layer "B.Cu") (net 1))
 (segment (start 139.4404 135.42) (end 151.3804 147.36) (width 0.25) (layer "F.Cu") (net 9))
 (segment (start 151.3804 147.36) (end 183.77 147.36) (width 0.25) (layer "F.Cu") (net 9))
 (segment (start 135 135) (end 135 140) (width 0.25) (layer "B.Cu") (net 10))
 (segment (start 137.12 132.88) (end 135 135) (width 0.25) (layer "B.Cu") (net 10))
 (segment (start 139.4404 132.88) (end 137.12 132.88) (width 0.25) (layer "B.Cu") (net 10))
 (segment (start 139.82 144.82) (end 183.77 144.82) (width 0.25) (layer "B.Cu") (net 10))
 (segment (start 135 140) (end 139.82 144.82) (width 0.25) (layer "B.Cu") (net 10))
 (segment (start 131.791391 77.92) (end 116 77.92) (width 0.25) (layer "B.Cu") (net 3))
 (segment (start 154.6804 120.18) (end 155.82 120.18) (width 0.25) (layer "B.Cu") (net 3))
 (segment (start 159 105.128609) (end 131.791391 77.92) (width 0.25) (layer "B.Cu") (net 3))
 (segment (start 155.82 120.18) (end 159 117) (width 0.25) (layer "B.Cu") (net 3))
 (segment (start 159 117) (end 159 105.128609) (width 0.25) (layer "B.Cu") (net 3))
 (segment (start 152 64.08) (end 152 84) (width 0.25) (layer "F.Cu") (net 8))
 (segment (start 114.9548 102.146) (end 113.1768 103.924) (width 0.25) (layer "F.Cu") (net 8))
 (segment (start 113.1768 114.9476) (end 115.92 117.6908) (width 0.25) (layer "F.Cu") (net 8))
 (segment (start 152 84) (end 152 99.7196) (width 0.25) (layer "F.Cu") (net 8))
 (segment (start 115.9708 102.146) (end 114.9548 102.146) (width 0.25) (layer "F.Cu") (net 8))
 (segment (start 133.854 102.146) (end 152 84) (width 0.25) (layer "F.Cu") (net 8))
 (segment (start 154.6804 102.4) (end 153.1402 100.8598) (width 0.25) (layer "F.Cu") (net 8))
 (segment (start 113.1768 103.924) (end 113.1768 114.9476) (width 0.25) (layer "F.Cu") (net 8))
 (segment (start 152 99.7196) (end 153.1402 100.8598) (width 0.25) (layer "F.Cu") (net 8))
 (segment (start 115.9708 102.146) (end 133.854 102.146) (width 0.25) (layer "F.Cu") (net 8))
 (segment (start 121.6604 104.94) (end 139.4404 104.94) (width 0.25) (layer "F.Cu") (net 7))
 (segment (start 121.5588 104.8384) (end 118.3584 104.8384) (width 0.25) (layer "F.Cu") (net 7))
 (segment (start 118.3584 104.8384) (end 115.9708 107.226) (width 0.25) (layer "F.Cu") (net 7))
 (segment (start 121.5588 104.8384) (end 121.6604 104.94) (width 0.25) (layer "F.Cu") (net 7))
 (segment (start 121.6096 111.6456) (end 125.7752 107.48) (width 0.25) (layer "F.Cu") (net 16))
 (segment (start 121.5588 111.6456) (end 121.6096 111.6456) (width 0.25) (layer "F.Cu") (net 16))
 (segment (start 119.476 111.6456) (end 117.5964 109.766) (width 0.25) (layer "F.Cu") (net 16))
 (segment (start 121.5588 111.6456) (end 119.476 111.6456) (width 0.25) (layer "F.Cu") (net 16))
 (segment (start 117.5964 109.766) (end 115.9708 109.766) (width 0.25) (layer "F.Cu") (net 16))
 (segment (start 125.7752 107.48) (end 139.4404 107.48) (width 0.25) (layer "F.Cu") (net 16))
 (segment (start 122.0668 120.2976) (end 132.3444 110.02) (width 0.25) (layer "F.Cu") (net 17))
 (segment (start 122.0668 120.2976) (end 118.3932 120.2976) (width 0.25) (layer "F.Cu") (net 17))
 (segment (start 118.3932 120.2976) (end 115.92 122.7708) (width 0.25) (layer "F.Cu") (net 17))
 (segment (start 132.3444 110.02) (end 139.4404 110.02) (width 0.25) (layer "F.Cu") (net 17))
 (segment (start 122.0668 127.2092) (end 117.8184 127.2092) (width 0.25) (layer "F.Cu") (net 18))
 (segment (start 122.0668 127.2092) (end 124.6896 127.2092) (width 0.25) (layer "F.Cu") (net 18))
 (segment (start 139.3388 112.56) (end 139.4404 112.56) (width 0.25) (layer "F.Cu") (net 18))
 (segment (start 117.8184 127.2092) (end 115.92 125.3108) (width 0.25) (layer "F.Cu") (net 18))
 (segment (start 124.6896 127.2092) (end 139.3388 112.56) (width 0.25) (layer "F.Cu") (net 18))
 (segment (start 173 108.13) (end 183.77 97.36) (width 0.25) (layer "F.Cu") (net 32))
 (segment (start 173 114.5604) (end 173 108.13) (width 0.25) (layer "F.Cu") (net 32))
 (segment (start 154.6804 132.88) (end 173 114.5604) (width 0.25) (layer "F.Cu") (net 32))
 (segment (start 154.6804 135.42) (end 157.58 135.42) (width 0.25) (layer "B.Cu") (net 31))
 (segment (start 166 127) (end 166 112.59) (width 0.25) (layer "B.Cu") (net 31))
 (segment (start 157.58 135.42) (end 166 127) (width 0.25) (layer "B.Cu") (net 31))
 (segment (start 166 112.59) (end 183.77 94.82) (width 0.25) (layer "B.Cu") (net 31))
 (segment (start 156 55) (end 167.46 55) (width 0.25) (layer "F.Cu") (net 5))
 (segment (start 152 59) (end 156 55) (width 0.25) (layer "F.Cu") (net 5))
 (segment (start 148 55) (end 152 59) (width 0.25) (layer "F.Cu") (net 5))
 (segment (start 126.54 55) (end 148 55) (width 0.25) (layer "F.Cu") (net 5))
 (segment (start 200 55) (end 227 82) (width 0.25) (layer "F.Cu") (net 6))
 (segment (start 170 55) (end 200 55) (width 0.25) (layer "F.Cu") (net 6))
 (segment (start 227 82) (end 227 115) (width 0.25) (layer "F.Cu") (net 6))
 (segment (start 131.38 75.38) (end 116 75.38) (width 0.25) (layer "B.Cu") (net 4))
 (segment (start 160 117.4004) (end 160 104) (width 0.25) (layer "B.Cu") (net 4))
 (segment (start 154.6804 122.72) (end 160 117.4004) (width 0.25) (layer "B.Cu") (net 4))
 (segment (start 160 104) (end 131.38 75.38) (width 0.25) (layer "B.Cu") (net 4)))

